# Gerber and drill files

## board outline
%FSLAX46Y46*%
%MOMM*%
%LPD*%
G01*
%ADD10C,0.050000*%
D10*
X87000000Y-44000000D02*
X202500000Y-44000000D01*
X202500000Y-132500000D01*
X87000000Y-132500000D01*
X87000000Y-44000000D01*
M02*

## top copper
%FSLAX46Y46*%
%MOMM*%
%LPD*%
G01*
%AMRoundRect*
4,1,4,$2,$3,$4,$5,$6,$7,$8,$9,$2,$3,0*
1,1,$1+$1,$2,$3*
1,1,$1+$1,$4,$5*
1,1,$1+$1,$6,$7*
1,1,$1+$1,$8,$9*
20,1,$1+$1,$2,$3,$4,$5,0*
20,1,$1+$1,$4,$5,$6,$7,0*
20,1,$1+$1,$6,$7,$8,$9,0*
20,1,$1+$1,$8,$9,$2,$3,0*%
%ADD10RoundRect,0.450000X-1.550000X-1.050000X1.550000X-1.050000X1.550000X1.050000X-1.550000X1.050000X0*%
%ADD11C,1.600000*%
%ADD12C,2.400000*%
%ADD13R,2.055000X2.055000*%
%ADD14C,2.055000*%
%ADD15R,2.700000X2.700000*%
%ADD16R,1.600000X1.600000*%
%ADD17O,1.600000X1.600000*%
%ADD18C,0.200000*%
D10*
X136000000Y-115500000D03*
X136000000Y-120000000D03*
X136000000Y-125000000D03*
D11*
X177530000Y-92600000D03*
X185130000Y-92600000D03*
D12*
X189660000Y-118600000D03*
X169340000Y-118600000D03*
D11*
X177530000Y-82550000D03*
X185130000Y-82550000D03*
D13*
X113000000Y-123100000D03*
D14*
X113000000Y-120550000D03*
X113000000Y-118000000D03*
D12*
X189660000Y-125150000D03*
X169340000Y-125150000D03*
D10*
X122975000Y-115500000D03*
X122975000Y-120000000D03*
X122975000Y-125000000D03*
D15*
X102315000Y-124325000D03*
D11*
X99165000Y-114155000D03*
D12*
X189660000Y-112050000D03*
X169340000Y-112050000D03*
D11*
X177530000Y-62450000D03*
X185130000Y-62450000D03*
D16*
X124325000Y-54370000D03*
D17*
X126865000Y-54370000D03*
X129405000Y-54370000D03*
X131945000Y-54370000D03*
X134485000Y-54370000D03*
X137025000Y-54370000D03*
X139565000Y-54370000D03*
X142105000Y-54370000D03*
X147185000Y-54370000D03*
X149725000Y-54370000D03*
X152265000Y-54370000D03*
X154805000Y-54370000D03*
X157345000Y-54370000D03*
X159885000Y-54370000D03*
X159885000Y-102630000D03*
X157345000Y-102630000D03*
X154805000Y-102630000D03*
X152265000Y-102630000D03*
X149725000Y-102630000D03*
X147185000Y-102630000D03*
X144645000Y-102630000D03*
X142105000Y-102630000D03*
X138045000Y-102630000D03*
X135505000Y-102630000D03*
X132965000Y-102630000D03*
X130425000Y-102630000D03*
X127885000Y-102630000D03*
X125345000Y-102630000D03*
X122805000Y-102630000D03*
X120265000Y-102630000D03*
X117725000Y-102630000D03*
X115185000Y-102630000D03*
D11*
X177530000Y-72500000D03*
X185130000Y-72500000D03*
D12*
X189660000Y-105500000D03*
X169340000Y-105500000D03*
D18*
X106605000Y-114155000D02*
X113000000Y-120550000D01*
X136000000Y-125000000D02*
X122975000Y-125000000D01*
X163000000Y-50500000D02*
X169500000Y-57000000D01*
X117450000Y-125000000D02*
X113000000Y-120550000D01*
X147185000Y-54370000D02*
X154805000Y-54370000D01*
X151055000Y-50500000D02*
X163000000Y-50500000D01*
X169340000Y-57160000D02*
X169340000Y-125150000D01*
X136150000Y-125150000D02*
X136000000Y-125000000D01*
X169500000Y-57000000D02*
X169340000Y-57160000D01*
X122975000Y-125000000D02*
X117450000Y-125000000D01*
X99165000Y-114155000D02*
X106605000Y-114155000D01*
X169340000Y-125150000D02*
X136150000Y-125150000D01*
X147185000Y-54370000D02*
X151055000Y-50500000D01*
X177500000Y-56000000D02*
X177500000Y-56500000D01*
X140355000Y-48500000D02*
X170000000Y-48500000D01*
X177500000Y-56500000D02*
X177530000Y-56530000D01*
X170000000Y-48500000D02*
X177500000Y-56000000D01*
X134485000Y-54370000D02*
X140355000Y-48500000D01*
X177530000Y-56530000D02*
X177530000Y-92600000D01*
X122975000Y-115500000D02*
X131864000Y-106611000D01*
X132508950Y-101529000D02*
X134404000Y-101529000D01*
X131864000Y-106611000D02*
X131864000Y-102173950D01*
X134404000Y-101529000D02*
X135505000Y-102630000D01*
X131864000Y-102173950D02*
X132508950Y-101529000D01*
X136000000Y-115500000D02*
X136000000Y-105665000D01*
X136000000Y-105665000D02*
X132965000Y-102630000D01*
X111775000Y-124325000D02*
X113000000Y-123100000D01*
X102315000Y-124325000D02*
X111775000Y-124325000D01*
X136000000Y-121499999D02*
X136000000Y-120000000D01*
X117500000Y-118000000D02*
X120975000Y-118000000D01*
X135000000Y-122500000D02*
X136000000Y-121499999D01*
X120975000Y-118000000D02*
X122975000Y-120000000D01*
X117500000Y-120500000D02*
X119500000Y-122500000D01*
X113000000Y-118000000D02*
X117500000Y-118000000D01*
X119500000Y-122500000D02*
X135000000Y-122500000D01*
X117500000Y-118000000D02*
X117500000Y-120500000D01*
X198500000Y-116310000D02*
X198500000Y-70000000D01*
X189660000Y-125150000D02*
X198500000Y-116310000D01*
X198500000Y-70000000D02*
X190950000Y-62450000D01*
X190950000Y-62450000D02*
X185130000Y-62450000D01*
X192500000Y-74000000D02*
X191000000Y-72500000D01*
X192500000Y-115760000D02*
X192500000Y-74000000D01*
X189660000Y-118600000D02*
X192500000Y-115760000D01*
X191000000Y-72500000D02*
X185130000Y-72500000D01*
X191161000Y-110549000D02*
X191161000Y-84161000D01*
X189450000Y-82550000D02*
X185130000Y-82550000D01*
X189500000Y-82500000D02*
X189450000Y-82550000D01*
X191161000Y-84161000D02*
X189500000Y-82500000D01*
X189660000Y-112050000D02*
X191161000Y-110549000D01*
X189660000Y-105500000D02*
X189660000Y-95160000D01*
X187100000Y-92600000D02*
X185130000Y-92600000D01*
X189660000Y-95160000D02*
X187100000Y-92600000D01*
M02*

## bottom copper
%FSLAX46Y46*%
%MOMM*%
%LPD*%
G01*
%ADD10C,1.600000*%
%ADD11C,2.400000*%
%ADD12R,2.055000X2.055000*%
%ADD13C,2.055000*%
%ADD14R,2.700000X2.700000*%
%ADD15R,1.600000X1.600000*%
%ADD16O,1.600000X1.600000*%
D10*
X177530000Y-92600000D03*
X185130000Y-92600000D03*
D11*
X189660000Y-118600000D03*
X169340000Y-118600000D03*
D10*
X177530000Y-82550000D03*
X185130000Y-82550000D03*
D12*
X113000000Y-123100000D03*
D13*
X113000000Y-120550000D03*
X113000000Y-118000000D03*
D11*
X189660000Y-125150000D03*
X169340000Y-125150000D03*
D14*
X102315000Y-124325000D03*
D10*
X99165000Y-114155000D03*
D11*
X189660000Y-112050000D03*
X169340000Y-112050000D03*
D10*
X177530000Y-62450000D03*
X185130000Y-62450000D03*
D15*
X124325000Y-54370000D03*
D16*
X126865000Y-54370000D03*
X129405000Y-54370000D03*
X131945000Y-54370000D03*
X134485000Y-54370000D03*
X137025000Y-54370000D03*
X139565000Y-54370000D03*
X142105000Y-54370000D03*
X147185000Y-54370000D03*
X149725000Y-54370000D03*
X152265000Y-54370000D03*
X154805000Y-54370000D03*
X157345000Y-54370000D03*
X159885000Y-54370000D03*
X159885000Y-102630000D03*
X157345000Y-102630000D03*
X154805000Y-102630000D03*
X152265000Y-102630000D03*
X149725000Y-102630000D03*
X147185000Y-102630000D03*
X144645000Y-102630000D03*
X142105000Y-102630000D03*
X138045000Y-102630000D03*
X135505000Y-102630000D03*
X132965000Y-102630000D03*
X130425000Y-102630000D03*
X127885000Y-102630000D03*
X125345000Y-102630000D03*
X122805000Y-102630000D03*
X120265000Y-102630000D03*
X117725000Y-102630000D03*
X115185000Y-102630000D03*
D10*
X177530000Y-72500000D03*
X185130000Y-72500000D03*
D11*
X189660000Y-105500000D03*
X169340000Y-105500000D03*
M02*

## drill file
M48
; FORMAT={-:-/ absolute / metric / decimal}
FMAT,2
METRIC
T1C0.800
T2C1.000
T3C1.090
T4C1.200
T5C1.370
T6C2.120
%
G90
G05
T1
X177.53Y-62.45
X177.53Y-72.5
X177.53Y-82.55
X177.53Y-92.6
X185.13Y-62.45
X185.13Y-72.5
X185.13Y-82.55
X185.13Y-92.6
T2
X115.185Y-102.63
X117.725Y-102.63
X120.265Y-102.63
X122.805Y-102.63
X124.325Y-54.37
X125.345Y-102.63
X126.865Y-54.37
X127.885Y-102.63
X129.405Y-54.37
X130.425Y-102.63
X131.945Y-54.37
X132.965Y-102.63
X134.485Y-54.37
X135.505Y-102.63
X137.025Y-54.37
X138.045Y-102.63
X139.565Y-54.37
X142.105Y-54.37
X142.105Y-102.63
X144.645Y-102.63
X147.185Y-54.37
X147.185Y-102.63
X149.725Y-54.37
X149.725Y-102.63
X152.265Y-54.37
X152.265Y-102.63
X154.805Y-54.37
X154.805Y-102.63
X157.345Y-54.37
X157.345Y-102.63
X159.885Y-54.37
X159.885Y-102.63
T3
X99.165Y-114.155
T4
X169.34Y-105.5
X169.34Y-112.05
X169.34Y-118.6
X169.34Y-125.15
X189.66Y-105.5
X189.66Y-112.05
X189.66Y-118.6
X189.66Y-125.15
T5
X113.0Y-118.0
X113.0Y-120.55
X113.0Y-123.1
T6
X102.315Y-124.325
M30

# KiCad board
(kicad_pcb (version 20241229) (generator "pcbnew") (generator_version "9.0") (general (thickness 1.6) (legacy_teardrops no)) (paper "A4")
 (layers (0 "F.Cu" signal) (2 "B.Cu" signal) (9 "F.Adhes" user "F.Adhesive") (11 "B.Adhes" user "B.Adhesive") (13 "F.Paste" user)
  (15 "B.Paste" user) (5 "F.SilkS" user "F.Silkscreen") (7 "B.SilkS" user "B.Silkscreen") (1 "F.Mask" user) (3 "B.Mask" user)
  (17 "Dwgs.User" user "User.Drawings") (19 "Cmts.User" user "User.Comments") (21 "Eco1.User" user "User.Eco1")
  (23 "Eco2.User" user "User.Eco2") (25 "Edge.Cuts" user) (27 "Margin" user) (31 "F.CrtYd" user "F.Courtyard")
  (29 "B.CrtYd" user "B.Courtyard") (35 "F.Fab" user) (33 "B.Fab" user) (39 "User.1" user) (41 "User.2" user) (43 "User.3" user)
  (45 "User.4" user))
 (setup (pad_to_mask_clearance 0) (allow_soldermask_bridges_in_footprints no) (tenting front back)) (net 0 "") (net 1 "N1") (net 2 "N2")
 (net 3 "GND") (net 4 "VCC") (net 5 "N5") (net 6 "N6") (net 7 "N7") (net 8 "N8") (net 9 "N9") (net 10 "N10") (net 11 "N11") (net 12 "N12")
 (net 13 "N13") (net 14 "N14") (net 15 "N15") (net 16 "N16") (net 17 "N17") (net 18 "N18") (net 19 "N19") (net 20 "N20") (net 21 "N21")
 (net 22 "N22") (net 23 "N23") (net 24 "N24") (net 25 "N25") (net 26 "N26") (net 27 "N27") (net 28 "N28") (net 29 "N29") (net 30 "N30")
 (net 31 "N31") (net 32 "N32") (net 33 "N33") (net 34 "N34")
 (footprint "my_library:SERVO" (layer "F.Cu") (at 136 122)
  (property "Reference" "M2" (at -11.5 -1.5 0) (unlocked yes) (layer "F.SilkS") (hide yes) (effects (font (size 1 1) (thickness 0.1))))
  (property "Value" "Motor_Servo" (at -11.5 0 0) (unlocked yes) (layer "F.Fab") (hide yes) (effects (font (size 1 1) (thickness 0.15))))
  (pad "1" smd roundrect (at 0 -6.5) (size 4 3) (layers "F.Cu" "F.Mask" "F.Paste") (roundrect_rratio 0.15) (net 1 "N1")
   (thermal_bridge_angle 45))
  (pad "2" smd roundrect (at 0 -2) (size 4 3) (layers "F.Cu" "F.Mask" "F.Paste") (roundrect_rratio 0.15) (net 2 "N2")
   (thermal_bridge_angle 45))
  (pad "3" smd roundrect (at 0 3) (size 4 3) (layers "F.Cu" "F.Mask" "F.Paste") (roundrect_rratio 0.15) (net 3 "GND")
   (thermal_bridge_angle 45)))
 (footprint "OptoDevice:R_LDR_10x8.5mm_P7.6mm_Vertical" (layer "F.Cu") (at 177.53 92.6)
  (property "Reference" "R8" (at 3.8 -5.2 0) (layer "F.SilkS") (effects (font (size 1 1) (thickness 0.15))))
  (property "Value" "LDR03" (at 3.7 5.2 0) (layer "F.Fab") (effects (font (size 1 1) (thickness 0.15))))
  (pad "1" thru_hole circle (at 0 0) (size 1.6 1.6) (drill 0.8) (layers "*.Cu" "*.Mask") (remove_unused_layers no) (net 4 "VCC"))
  (pad "2" thru_hole circle (at 7.6 0) (size 1.6 1.6) (drill 0.8) (layers "*.Cu" "*.Mask") (remove_unused_layers no) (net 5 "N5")))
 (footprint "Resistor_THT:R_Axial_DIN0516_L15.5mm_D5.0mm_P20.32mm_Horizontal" (layer "F.Cu") (at 189.66 118.6 180)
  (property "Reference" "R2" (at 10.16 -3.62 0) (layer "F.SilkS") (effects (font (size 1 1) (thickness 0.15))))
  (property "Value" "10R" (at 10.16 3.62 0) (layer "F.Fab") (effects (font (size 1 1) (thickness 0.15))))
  (pad "1" thru_hole circle (at 0 0 180) (size 2.4 2.4) (drill 1.2) (layers "*.Cu" "*.Mask") (remove_unused_layers no) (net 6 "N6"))
  (pad "2" thru_hole circle (at 20.32 0 180) (size 2.4 2.4) (drill 1.2) (layers "*.Cu" "*.Mask") (remove_unused_layers no) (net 3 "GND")))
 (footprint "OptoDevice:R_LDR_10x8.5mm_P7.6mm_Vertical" (layer "F.Cu") (at 177.53 82.55)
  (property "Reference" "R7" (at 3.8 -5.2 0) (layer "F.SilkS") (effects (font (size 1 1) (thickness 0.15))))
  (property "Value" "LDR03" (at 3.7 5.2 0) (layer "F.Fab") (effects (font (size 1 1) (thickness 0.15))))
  (pad "1" thru_hole circle (at 0 0) (size 1.6 1.6) (drill 0.8) (layers "*.Cu" "*.Mask") (remove_unused_layers no) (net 4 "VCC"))
  (pad "2" thru_hole circle (at 7.6 0) (size 1.6 1.6) (drill 0.8) (layers "*.Cu" "*.Mask") (remove_unused_layers no) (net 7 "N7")))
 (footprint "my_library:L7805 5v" (layer "F.Cu") (at 112.3375 120.55 90)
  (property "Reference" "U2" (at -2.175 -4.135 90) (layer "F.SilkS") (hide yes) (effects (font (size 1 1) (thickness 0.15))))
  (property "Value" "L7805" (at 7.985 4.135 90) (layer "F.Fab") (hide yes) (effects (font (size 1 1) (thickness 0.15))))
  (pad "1" thru_hole rect (at -2.55 0.6625 90) (size 2.055 2.055) (drill 1.37) (layers "*.Cu" "*.Mask") (remove_unused_layers no)
   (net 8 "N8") (solder_mask_margin 0.102))
  (pad "2" thru_hole circle (at 0 0.6625 90) (size 2.055 2.055) (drill 1.37) (layers "*.Cu" "*.Mask") (remove_unused_layers no)
   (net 3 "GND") (solder_mask_margin 0.102))
  (pad "3" thru_hole circle (at 2.55 0.6625 90) (size 2.055 2.055) (drill 1.37) (layers "*.Cu" "*.Mask") (remove_unused_layers no)
   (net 2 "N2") (solder_mask_margin 0.102)))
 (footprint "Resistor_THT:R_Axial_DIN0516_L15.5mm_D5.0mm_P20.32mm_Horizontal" (layer "F.Cu") (at 189.66 125.15 180)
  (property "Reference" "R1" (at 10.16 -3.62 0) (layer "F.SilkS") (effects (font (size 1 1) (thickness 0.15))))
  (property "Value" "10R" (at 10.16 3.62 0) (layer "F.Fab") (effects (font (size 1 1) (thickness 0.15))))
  (pad "1" thru_hole circle (at 0 0 180) (size 2.4 2.4) (drill 1.2) (layers "*.Cu" "*.Mask") (remove_unused_layers no) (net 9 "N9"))
  (pad "2" thru_hole circle (at 20.32 0 180) (size 2.4 2.4) (drill 1.2) (layers "*.Cu" "*.Mask") (remove_unused_layers no) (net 3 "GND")))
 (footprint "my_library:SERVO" (layer "F.Cu") (at 122.975 122)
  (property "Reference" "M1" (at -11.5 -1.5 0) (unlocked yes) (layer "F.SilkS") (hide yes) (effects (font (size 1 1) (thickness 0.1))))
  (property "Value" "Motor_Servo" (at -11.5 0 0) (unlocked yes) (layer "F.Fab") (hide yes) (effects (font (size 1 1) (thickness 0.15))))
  (pad "1" smd roundrect (at 0 -6.5) (size 4 3) (layers "F.Cu" "F.Mask" "F.Paste") (roundrect_rratio 0.15) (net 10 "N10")
   (thermal_bridge_angle 45))
  (pad "2" smd roundrect (at 0 -2) (size 4 3) (layers "F.Cu" "F.Mask" "F.Paste") (roundrect_rratio 0.15) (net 2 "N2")
   (thermal_bridge_angle 45))
  (pad "3" smd roundrect (at 0 3) (size 4 3) (layers "F.Cu" "F.Mask" "F.Paste") (roundrect_rratio 0.15) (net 3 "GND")
   (thermal_bridge_angle 45)))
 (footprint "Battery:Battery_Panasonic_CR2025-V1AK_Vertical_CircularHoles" (layer "F.Cu") (at 102.315 124.325 90)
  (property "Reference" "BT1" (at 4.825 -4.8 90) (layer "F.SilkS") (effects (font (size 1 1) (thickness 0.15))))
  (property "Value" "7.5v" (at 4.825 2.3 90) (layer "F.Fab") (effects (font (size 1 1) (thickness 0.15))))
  (pad "1" thru_hole rect (at 0 0 180) (size 2.7 2.7) (drill 2.12) (layers "*.Cu" "*.Mask") (remove_unused_layers no) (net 8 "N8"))
  (pad "2" thru_hole circle (at 10.17 -3.15 90) (size 1.6 1.6) (drill 1.09) (layers "*.Cu" "*.Mask") (remove_unused_layers no) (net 3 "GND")))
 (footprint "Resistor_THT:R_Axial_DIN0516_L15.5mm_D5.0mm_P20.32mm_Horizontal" (layer "F.Cu") (at 189.66 112.05 180)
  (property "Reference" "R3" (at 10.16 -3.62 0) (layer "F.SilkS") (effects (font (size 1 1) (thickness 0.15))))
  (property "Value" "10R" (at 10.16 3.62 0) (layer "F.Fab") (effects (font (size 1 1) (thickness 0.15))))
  (pad "1" thru_hole circle (at 0 0 180) (size 2.4 2.4) (drill 1.2) (layers "*.Cu" "*.Mask") (remove_unused_layers no) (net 7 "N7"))
  (pad "2" thru_hole circle (at 20.32 0 180) (size 2.4 2.4) (drill 1.2) (layers "*.Cu" "*.Mask") (remove_unused_layers no) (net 3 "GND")))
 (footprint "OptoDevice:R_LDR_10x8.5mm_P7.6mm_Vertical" (layer "F.Cu") (at 177.53 62.45)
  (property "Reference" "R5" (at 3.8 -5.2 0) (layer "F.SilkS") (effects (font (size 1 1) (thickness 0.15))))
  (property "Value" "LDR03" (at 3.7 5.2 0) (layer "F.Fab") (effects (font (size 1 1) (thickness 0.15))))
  (pad "1" thru_hole circle (at 0 0) (size 1.6 1.6) (drill 0.8) (layers "*.Cu" "*.Mask") (remove_unused_layers no) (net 4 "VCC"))
  (pad "2" thru_hole circle (at 7.6 0) (size 1.6 1.6) (drill 0.8) (layers "*.Cu" "*.Mask") (remove_unused_layers no) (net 9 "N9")))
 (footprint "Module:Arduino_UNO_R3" (layer "F.Cu") (at 124.325 54.37)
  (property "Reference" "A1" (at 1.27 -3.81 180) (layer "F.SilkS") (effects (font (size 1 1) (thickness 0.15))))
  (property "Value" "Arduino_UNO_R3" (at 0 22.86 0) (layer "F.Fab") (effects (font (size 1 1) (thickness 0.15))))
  (pad "1" thru_hole rect (at 0 0 90) (size 1.6 1.6) (drill 1) (layers "*.Cu" "*.Mask") (remove_unused_layers no) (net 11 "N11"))
  (pad "2" thru_hole oval (at 2.54 0 90) (size 1.6 1.6) (drill 1) (layers "*.Cu" "*.Mask") (remove_unused_layers no) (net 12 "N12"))
  (pad "3" thru_hole oval (at 5.08 0 90) (size 1.6 1.6) (drill 1) (layers "*.Cu" "*.Mask") (remove_unused_layers no) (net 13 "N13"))
  (pad "4" thru_hole oval (at 7.62 0 90) (size 1.6 1.6) (drill 1) (layers "*.Cu" "*.Mask") (remove_unused_layers no) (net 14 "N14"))
  (pad "5" thru_hole oval (at 10.16 0 90) (size 1.6 1.6) (drill 1) (layers "*.Cu" "*.Mask") (remove_unused_layers no) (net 4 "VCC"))
  (pad "6" thru_hole oval (at 12.7 0 90) (size 1.6 1.6) (drill 1) (layers "*.Cu" "*.Mask") (remove_unused_layers no) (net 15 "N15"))
  (pad "7" thru_hole oval (at 15.24 0 90) (size 1.6 1.6) (drill 1) (layers "*.Cu" "*.Mask") (remove_unused_layers no) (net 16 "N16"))
  (pad "8" thru_hole oval (at 17.78 0 90) (size 1.6 1.6) (drill 1) (layers "*.Cu" "*.Mask") (remove_unused_layers no) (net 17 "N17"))
  (pad "9" thru_hole oval (at 22.86 0 90) (size 1.6 1.6) (drill 1) (layers "*.Cu" "*.Mask") (remove_unused_layers no) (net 3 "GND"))
  (pad "10" thru_hole oval (at 25.4 0 90) (size 1.6 1.6) (drill 1) (layers "*.Cu" "*.Mask") (remove_unused_layers no) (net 3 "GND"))
  (pad "11" thru_hole oval (at 27.94 0 90) (size 1.6 1.6) (drill 1) (layers "*.Cu" "*.Mask") (remove_unused_layers no) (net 3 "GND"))
  (pad "12" thru_hole oval (at 30.48 0 90) (size 1.6 1.6) (drill 1) (layers "*.Cu" "*.Mask") (remove_unused_layers no) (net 3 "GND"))
  (pad "13" thru_hole oval (at 33.02 0 90) (size 1.6 1.6) (drill 1) (layers "*.Cu" "*.Mask") (remove_unused_layers no) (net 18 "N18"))
  (pad "14" thru_hole oval (at 35.56 0 90) (size 1.6 1.6) (drill 1) (layers "*.Cu" "*.Mask") (remove_unused_layers no) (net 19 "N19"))
  (pad "15" thru_hole oval (at 35.56 48.26 90) (size 1.6 1.6) (drill 1) (layers "*.Cu" "*.Mask") (remove_unused_layers no) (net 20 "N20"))
  (pad "16" thru_hole oval (at 33.02 48.26 90) (size 1.6 1.6) (drill 1) (layers "*.Cu" "*.Mask") (remove_unused_layers no) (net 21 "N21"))
  (pad "17" thru_hole oval (at 30.48 48.26 90) (size 1.6 1.6) (drill 1) (layers "*.Cu" "*.Mask") (remove_unused_layers no) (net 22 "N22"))
  (pad "18" thru_hole oval (at 27.94 48.26 90) (size 1.6 1.6) (drill 1) (layers "*.Cu" "*.Mask") (remove_unused_layers no) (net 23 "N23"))
  (pad "19" thru_hole oval (at 25.4 48.26 90) (size 1.6 1.6) (drill 1) (layers "*.Cu" "*.Mask") (remove_unused_layers no) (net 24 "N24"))
  (pad "20" thru_hole oval (at 22.86 48.26 90) (size 1.6 1.6) (drill 1) (layers "*.Cu" "*.Mask") (remove_unused_layers no) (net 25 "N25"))
  (pad "21" thru_hole oval (at 20.32 48.26 90) (size 1.6 1.6) (drill 1) (layers "*.Cu" "*.Mask") (remove_unused_layers no) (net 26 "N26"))
  (pad "22" thru_hole oval (at 17.78 48.26 90) (size 1.6 1.6) (drill 1) (layers "*.Cu" "*.Mask") (remove_unused_layers no) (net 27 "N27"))
  (pad "23" thru_hole oval (at 13.72 48.26 90) (size 1.6 1.6) (drill 1) (layers "*.Cu" "*.Mask") (remove_unused_layers no) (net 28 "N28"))
  (pad "24" thru_hole oval (at 11.18 48.26 90) (size 1.6 1.6) (drill 1) (layers "*.Cu" "*.Mask") (remove_unused_layers no) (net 10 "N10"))
  (pad "25" thru_hole oval (at 8.64 48.26 90) (size 1.6 1.6) (drill 1) (layers "*.Cu" "*.Mask") (remove_unused_layers no) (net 1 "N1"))
  (pad "26" thru_hole oval (at 6.1 48.26 90) (size 1.6 1.6) (drill 1) (layers "*.Cu" "*.Mask") (remove_unused_layers no) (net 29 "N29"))
  (pad "27" thru_hole oval (at 3.56 48.26 90) (size 1.6 1.6) (drill 1) (layers "*.Cu" "*.Mask") (remove_unused_layers no) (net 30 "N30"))
  (pad "28" thru_hole oval (at 1.02 48.26 90) (size 1.6 1.6) (drill 1) (layers "*.Cu" "*.Mask") (remove_unused_layers no) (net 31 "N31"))
  (pad "29" thru_hole oval (at -1.52 48.26 90) (size 1.6 1.6) (drill 1) (layers "*.Cu" "*.Mask") (remove_unused_layers no) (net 3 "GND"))
  (pad "30" thru_hole oval (at -4.06 48.26 90) (size 1.6 1.6) (drill 1) (layers "*.Cu" "*.Mask") (remove_unused_layers no) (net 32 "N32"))
  (pad "31" thru_hole oval (at -6.6 48.26 90) (size 1.6 1.6) (drill 1) (layers "*.Cu" "*.Mask") (remove_unused_layers no) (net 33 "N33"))
  (pad "32" thru_hole oval (at -9.14 48.26 90) (size 1.6 1.6) (drill 1) (layers "*.Cu" "*.Mask") (remove_unused_layers no) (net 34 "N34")))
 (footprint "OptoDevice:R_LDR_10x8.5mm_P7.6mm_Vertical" (layer "F.Cu") (at 177.53 72.5)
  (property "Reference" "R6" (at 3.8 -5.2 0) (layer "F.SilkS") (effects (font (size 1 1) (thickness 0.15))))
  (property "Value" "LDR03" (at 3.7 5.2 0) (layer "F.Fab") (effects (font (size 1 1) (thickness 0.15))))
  (pad "1" thru_hole circle (at 0 0) (size 1.6 1.6) (drill 0.8) (layers "*.Cu" "*.Mask") (remove_unused_layers no) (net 4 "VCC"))
  (pad "2" thru_hole circle (at 7.6 0) (size 1.6 1.6) (drill 0.8) (layers "*.Cu" "*.Mask") (remove_unused_layers no) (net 6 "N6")))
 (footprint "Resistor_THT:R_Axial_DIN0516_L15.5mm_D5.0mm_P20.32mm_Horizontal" (layer "F.Cu") (at 189.66 105.5 180)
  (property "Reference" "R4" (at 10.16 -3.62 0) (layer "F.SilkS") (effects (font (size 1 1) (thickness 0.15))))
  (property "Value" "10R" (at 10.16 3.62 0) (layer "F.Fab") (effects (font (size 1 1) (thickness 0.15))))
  (pad "1" thru_hole circle (at 0 0 180) (size 2.4 2.4) (drill 1.2) (layers "*.Cu" "*.Mask") (remove_unused_layers no) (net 5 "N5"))
  (pad "2" thru_hole circle (at 20.32 0 180) (size 2.4 2.4) (drill 1.2) (layers "*.Cu" "*.Mask") (remove_unused_layers no) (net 3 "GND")))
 (gr_rect (start 87 44) (end 202.5 132.5) (stroke (width 0.05) (type default)) (fill no) (layer "Edge.Cuts"))
 (segment (start 106.605 114.155) (end 113 120.55) (width 0.2) (layer "F.Cu") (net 3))
 (segment (start 136 125) (end 122.975 125) (width 0.2) (layer "F.Cu") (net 3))
 (segment (start 163 50.5) (end 169.5 57) (width 0.2) (layer "F.Cu") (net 3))
 (segment (start 117.45 125) (end 113 120.55) (width 0.2) (layer "F.Cu") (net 3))
 (segment (start 147.185 54.37) (end 154.805 54.37) (width 0.2) (layer "F.Cu") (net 3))
 (segment (start 151.055 50.5) (end 163 50.5) (width 0.2) (layer "F.Cu") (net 3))
 (segment (start 169.34 57.16) (end 169.34 125.15) (width 0.2) (layer "F.Cu") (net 3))
 (segment (start 136.15 125.15) (end 136 125) (width 0.2) (layer "F.Cu") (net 3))
 (segment (start 169.5 57) (end 169.34 57.16) (width 0.2) (layer "F.Cu") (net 3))
 (segment (start 122.975 125) (end 117.45 125) (width 0.2) (layer "F.Cu") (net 3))
 (segment (start 99.165 114.155) (end 106.605 114.155) (width 0.2) (layer "F.Cu") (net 3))
 (segment (start 169.34 125.15) (end 136.15 125.15) (width 0.2) (layer "F.Cu") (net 3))
 (segment (start 147.185 54.37) (end 151.055 50.5) (width 0.2) (layer "F.Cu") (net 3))
 (segment (start 177.5 56) (end 177.5 56.5) (width 0.2) (layer "F.Cu") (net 4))
 (segment (start 140.355 48.5) (end 170 48.5) (width 0.2) (layer "F.Cu") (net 4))
 (segment (start 177.5 56.5) (end 177.53 56.53) (width 0.2) (layer "F.Cu") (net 4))
 (segment (start 170 48.5) (end 177.5 56) (width 0.2) (layer "F.Cu") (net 4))
 (segment (start 134.485 54.37) (end 140.355 48.5) (width 0.2) (layer "F.Cu") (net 4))
 (segment (start 177.53 56.53) (end 177.53 92.6) (width 0.2) (layer "F.Cu") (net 4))
 (segment (start 122.975 115.5) (end 131.864 106.611) (width 0.2) (layer "F.Cu") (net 10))
 (segment (start 132.50895 101.529) (end 134.404 101.529) (width 0.2) (layer "F.Cu") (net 10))
 (segment (start 131.864 106.611) (end 131.864 102.17395) (width 0.2) (layer "F.Cu") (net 10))
 (segment (start 134.404 101.529) (end 135.505 102.63) (width 0.2) (layer "F.Cu") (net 10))
 (segment (start 131.864 102.17395) (end 132.50895 101.529) (width 0.2) (layer "F.Cu") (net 10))
 (segment (start 136 115.5) (end 136 105.665) (width 0.2) (layer "F.Cu") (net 1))
 (segment (start 136 105.665) (end 132.965 102.63) (width 0.2) (layer "F.Cu") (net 1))
 (segment (start 111.775 124.325) (end 113 123.1) (width 0.2) (layer "F.Cu") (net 8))
 (segment (start 102.315 124.325) (end 111.775 124.325) (width 0.2) (layer "F.Cu") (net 8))
 (segment (start 136 121.499999) (end 136 120) (width 0.2) (layer "F.Cu") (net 2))
 (segment (start 117.5 118) (end 120.975 118) (width 0.2) (layer "F.Cu") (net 2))
 (segment (start 135 122.5) (end 136 121.499999) (width 0.2) (layer "F.Cu") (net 2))
 (segment (start 120.975 118) (end 122.975 120) (width 0.2) (layer "F.Cu") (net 2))
 (segment (start 117.5 120.5) (end 119.5 122.5) (width 0.2) (layer "F.Cu") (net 2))
 (segment (start 113 118) (end 117.5 118) (width 0.2) (layer "F.Cu") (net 2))
 (segment (start 119.5 122.5) (end 135 122.5) (width 0.2) (layer "F.Cu") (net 2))
 (segment (start 117.5 118) (end 117.5 120.5) (width 0.2) (layer "F.Cu") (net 2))
 (segment (start 198.5 116.31) (end 198.5 70) (width 0.2) (layer "F.Cu") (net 9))
 (segment (start 189.66 125.15) (end 198.5 116.31) (width 0.2) (layer "F.Cu") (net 9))
 (segment (start 198.5 70) (end 190.95 62.45) (width 0.2) (layer "F.Cu") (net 9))
 (segment (start 190.95 62.45) (end 185.13 62.45) (width 0.2) (layer "F.Cu") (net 9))
 (segment (start 192.5 74) (end 191 72.5) (width 0.2) (layer "F.Cu") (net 6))
 (segment (start 192.5 115.76) (end 192.5 74) (width 0.2) (layer "F.Cu") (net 6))
 (segment (start 189.66 118.6) (end 192.5 115.76) (width 0.2) (layer "F.Cu") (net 6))
 (segment (start 191 72.5) (end 185.13 72.5) (width 0.2) (layer "F.Cu") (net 6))
 (segment (start 191.161 110.549) (end 191.161 84.161) (width 0.2) (layer "F.Cu") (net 7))
 (segment (start 189.45 82.55) (end 185.13 82.55) (width 0.2) (layer "F.Cu") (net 7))
 (segment (start 189.5 82.5) (end 189.45 82.55) (width 0.2) (layer "F.Cu") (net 7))
 (segment (start 191.161 84.161) (end 189.5 82.5) (width 0.2) (layer "F.Cu") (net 7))
 (segment (start 189.66 112.05) (end 191.161 110.549) (width 0.2) (layer "F.Cu") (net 7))
 (segment (start 189.66 105.5) (end 189.66 95.16) (width 0.2) (layer "F.Cu") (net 5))
 (segment (start 187.1 92.6) (end 185.13 92.6) (width 0.2) (layer "F.Cu") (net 5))
 (segment (start 189.66 95.16) (end 187.1 92.6) (width 0.2) (layer "F.Cu") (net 5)))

